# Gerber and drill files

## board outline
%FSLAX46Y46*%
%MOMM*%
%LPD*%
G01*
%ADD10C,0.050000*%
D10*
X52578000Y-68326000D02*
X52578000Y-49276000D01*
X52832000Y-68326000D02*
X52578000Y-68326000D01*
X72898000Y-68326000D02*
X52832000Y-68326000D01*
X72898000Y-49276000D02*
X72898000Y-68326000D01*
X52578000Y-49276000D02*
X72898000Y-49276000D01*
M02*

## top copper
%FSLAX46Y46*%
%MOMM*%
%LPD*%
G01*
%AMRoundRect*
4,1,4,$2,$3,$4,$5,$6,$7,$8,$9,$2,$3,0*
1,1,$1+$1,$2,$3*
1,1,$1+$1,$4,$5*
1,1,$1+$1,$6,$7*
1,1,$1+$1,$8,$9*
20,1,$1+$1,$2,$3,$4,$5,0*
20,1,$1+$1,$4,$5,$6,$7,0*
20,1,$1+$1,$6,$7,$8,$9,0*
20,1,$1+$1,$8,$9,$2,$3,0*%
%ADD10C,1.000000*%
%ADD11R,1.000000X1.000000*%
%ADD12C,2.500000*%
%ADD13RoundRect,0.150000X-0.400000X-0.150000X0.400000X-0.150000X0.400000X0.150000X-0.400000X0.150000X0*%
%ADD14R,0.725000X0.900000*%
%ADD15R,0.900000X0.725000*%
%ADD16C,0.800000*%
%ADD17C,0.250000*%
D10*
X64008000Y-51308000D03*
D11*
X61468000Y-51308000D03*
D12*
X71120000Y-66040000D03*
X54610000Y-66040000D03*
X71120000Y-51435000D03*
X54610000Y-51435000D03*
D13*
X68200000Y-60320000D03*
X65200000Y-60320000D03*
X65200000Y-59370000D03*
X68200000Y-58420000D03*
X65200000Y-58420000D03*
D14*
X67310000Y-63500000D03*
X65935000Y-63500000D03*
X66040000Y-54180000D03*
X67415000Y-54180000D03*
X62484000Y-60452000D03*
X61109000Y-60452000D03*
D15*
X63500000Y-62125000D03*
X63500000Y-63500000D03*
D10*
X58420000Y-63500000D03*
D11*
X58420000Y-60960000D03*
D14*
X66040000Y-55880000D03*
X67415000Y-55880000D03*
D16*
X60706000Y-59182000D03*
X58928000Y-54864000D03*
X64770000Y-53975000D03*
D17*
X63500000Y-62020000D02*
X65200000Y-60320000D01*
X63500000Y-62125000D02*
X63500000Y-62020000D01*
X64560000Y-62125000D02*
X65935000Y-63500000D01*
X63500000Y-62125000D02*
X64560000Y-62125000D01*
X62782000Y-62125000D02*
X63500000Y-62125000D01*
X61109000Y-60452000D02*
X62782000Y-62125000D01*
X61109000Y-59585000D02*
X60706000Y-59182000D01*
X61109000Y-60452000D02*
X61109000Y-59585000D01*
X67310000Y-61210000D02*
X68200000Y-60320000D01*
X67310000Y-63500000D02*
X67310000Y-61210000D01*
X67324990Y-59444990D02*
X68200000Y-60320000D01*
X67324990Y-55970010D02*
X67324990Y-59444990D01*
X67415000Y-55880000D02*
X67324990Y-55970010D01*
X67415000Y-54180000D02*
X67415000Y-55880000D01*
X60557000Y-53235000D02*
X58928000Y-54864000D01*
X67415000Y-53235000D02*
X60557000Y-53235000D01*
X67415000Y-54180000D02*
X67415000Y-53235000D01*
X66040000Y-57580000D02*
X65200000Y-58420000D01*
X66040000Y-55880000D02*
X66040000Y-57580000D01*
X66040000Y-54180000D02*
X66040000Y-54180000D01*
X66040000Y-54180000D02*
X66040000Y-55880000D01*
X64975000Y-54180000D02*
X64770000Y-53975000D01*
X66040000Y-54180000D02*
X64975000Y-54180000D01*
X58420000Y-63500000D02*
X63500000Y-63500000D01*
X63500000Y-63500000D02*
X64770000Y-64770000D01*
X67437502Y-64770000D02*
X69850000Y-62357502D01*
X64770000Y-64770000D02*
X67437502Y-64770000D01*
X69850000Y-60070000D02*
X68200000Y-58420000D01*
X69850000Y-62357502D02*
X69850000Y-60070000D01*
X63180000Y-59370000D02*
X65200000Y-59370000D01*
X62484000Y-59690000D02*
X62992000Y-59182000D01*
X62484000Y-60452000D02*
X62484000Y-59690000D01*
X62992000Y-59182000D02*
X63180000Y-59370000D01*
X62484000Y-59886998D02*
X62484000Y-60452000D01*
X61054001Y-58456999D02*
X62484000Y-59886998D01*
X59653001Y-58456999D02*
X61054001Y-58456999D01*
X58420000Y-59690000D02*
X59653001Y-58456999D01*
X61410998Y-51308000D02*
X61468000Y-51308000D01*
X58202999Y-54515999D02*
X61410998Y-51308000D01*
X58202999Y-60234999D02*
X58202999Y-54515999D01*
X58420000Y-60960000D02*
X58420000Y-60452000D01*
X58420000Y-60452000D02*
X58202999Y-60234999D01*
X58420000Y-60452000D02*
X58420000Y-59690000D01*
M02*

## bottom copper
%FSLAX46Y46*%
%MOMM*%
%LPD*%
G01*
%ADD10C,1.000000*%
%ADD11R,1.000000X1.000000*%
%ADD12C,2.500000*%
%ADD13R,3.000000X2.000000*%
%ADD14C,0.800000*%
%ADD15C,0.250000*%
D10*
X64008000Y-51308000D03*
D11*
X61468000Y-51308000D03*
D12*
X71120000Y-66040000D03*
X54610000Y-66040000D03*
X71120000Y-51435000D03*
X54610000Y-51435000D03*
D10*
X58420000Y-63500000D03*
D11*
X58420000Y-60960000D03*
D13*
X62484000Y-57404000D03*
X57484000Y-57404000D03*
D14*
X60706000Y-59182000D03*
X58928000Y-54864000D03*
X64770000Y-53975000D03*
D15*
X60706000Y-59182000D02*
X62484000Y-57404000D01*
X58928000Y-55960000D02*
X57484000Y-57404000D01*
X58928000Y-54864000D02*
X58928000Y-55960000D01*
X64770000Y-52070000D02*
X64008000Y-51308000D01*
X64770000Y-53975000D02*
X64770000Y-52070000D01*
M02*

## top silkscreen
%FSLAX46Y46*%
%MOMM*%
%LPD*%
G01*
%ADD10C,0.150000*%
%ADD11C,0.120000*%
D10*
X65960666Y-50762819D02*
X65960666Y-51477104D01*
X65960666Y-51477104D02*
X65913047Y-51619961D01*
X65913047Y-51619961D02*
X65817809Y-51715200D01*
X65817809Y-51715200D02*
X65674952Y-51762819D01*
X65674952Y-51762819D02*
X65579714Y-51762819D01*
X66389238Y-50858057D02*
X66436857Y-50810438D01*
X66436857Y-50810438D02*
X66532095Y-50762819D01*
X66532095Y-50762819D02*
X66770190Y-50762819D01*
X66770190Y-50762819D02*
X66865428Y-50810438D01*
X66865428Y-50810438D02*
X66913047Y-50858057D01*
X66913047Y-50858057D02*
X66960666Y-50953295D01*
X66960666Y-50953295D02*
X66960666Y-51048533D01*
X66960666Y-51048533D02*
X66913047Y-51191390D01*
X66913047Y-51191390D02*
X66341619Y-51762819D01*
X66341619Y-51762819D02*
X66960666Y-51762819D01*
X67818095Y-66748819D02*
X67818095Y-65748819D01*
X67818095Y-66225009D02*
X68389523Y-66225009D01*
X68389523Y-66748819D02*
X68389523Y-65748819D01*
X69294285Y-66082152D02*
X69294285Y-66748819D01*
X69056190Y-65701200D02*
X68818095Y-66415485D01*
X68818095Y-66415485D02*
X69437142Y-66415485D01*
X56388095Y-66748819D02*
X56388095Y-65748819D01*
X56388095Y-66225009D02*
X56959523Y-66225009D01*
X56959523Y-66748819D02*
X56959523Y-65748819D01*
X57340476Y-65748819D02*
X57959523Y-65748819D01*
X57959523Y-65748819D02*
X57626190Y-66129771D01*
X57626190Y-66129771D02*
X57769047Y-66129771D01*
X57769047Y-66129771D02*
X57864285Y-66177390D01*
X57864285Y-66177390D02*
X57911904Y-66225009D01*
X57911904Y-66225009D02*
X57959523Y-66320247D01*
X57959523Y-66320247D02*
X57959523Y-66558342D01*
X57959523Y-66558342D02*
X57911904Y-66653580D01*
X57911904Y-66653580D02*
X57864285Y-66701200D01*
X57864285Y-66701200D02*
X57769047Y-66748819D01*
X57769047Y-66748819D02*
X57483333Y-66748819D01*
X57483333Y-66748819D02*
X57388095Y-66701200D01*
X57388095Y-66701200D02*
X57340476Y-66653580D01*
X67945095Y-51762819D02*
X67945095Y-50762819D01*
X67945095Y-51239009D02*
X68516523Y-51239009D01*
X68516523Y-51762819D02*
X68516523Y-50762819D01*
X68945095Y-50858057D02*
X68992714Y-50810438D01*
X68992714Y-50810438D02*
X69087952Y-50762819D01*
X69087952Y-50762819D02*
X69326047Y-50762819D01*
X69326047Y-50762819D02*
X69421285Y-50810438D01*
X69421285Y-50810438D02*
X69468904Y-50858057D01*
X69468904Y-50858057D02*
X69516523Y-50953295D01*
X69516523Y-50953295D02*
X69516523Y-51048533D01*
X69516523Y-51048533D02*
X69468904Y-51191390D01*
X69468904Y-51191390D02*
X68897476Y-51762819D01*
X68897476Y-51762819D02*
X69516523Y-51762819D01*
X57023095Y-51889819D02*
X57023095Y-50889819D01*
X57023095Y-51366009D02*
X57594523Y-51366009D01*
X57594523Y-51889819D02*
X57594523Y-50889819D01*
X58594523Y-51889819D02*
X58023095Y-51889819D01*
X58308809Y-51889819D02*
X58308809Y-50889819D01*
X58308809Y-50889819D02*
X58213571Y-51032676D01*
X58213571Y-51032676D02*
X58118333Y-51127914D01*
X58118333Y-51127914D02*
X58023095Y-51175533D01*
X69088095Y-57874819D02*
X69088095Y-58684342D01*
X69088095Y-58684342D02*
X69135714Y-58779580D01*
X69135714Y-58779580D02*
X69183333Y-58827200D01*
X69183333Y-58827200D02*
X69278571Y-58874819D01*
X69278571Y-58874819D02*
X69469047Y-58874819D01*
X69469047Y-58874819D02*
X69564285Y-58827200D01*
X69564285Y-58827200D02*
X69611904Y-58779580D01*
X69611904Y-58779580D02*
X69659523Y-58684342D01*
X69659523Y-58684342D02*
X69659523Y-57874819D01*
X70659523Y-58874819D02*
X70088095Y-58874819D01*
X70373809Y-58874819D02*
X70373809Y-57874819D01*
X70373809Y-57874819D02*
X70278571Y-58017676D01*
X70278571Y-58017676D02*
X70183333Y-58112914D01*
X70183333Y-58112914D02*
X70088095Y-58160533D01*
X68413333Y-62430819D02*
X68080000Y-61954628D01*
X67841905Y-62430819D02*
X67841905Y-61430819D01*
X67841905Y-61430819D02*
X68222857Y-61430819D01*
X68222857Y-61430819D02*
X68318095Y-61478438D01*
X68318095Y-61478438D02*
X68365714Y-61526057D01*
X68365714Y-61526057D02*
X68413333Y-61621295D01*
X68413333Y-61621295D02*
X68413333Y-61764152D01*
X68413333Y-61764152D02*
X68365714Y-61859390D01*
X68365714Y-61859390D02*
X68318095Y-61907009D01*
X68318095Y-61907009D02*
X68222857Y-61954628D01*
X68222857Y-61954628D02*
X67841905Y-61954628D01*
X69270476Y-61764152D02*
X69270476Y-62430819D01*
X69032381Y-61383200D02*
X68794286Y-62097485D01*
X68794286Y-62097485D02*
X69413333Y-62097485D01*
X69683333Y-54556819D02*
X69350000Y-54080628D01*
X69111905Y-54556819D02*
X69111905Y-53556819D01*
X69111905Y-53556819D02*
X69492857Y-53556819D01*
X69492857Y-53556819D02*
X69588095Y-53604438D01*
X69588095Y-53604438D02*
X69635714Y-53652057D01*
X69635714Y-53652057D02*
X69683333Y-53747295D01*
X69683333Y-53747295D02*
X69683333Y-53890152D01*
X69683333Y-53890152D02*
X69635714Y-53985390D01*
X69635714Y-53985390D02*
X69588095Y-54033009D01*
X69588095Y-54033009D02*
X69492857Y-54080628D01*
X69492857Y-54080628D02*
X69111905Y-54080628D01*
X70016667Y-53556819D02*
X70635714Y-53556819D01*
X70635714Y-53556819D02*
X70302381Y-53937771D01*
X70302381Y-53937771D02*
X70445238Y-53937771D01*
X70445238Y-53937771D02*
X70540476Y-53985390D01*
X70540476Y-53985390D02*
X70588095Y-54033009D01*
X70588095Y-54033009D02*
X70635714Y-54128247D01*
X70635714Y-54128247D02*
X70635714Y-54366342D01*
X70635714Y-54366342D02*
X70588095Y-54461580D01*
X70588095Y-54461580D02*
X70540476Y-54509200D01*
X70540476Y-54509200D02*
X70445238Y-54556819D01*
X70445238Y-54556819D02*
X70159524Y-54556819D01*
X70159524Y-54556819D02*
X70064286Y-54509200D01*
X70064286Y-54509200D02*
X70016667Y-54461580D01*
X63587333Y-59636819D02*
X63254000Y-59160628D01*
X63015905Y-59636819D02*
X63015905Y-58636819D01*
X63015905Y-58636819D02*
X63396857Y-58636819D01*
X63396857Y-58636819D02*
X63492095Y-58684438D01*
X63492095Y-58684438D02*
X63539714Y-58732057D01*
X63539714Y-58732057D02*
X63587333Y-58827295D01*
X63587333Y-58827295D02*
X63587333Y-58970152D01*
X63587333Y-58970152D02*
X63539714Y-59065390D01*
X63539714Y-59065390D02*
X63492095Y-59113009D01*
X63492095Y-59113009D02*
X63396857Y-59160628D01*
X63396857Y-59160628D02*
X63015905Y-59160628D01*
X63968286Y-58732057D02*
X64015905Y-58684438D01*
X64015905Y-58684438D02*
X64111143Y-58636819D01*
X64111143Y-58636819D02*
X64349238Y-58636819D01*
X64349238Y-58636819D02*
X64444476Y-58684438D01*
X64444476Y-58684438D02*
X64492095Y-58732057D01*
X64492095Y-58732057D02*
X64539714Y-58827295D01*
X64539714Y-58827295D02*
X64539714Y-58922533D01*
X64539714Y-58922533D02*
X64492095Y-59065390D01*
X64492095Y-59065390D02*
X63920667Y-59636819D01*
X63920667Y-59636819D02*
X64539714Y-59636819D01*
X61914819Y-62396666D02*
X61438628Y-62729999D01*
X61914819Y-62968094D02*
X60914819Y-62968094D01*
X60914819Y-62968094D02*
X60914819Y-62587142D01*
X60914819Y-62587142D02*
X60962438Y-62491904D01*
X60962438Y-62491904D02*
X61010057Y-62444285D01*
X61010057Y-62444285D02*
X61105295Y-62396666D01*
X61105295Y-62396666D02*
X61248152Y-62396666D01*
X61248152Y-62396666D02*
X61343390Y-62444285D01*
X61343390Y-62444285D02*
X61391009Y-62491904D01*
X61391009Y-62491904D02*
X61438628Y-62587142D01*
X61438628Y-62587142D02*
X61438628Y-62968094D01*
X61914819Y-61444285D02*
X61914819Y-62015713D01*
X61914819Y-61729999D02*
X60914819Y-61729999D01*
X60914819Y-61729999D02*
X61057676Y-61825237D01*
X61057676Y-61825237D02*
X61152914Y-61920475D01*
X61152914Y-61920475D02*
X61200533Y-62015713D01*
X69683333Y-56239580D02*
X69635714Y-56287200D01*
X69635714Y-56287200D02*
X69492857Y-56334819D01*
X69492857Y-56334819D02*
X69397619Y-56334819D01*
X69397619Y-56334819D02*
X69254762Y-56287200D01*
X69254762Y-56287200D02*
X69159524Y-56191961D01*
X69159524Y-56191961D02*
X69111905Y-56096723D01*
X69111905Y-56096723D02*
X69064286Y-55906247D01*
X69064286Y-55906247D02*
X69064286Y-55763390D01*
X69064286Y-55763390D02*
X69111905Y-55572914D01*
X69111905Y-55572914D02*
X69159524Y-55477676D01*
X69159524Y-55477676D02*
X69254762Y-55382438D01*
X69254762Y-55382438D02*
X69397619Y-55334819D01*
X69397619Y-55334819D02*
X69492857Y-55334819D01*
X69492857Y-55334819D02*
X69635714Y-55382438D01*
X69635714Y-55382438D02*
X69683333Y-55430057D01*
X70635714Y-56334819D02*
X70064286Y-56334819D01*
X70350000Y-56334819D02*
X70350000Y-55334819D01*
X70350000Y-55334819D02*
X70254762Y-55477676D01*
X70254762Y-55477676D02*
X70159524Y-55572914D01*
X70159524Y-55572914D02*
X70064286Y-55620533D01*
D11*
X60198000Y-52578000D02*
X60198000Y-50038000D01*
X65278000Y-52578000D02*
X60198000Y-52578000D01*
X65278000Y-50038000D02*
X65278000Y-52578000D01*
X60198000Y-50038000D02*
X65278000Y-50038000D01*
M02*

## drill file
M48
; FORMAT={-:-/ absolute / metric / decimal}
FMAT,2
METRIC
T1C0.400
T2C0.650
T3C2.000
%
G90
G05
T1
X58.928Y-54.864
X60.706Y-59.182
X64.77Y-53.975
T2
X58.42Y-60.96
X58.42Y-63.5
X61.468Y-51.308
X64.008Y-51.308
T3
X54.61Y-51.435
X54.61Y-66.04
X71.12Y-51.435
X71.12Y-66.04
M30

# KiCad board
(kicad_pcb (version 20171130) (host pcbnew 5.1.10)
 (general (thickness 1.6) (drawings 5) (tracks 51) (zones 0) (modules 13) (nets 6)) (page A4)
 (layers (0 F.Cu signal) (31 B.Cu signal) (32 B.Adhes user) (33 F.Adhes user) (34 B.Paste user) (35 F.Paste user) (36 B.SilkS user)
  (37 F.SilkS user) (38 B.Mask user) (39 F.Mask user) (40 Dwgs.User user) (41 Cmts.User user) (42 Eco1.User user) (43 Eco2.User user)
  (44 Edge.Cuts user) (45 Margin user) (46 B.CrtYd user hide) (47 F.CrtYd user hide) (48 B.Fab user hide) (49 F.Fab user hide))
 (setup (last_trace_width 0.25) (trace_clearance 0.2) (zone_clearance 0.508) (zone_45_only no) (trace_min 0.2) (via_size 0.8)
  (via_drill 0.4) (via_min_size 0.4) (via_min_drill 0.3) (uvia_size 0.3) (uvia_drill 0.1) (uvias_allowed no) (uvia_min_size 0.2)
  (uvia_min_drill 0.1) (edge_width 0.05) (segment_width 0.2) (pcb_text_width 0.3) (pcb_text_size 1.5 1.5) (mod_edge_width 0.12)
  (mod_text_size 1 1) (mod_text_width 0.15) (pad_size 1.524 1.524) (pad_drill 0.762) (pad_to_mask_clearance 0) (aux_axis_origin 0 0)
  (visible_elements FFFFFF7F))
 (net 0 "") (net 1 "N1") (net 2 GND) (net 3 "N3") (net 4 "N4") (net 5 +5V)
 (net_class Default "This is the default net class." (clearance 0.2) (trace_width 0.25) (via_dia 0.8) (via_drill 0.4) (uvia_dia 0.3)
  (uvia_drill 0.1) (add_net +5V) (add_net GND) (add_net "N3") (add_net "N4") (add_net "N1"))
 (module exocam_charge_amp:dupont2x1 (layer F.Cu) (at 64.008 48.768)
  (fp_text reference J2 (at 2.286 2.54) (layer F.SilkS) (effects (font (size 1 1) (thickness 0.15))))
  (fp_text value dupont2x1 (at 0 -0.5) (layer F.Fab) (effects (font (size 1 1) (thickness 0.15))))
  (fp_line (start -3.81 3.81) (end -3.81 1.27) (layer F.SilkS) (width 0.12))
  (fp_line (start 1.27 3.81) (end -3.81 3.81) (layer F.SilkS) (width 0.12))
  (fp_line (start 1.27 1.27) (end 1.27 3.81) (layer F.SilkS) (width 0.12))
  (fp_line (start -3.81 1.27) (end 1.27 1.27) (layer F.SilkS) (width 0.12))
  (pad 2 thru_hole circle (at 0 2.54) (size 1 1) (drill 0.65) (layers *.Cu *.Mask) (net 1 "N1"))
  (pad 1 thru_hole rect (at -2.54 2.54) (size 1 1) (drill 0.65) (layers *.Cu *.Mask) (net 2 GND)))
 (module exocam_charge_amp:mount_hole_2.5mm (layer F.Cu) (at 72.39 62.23)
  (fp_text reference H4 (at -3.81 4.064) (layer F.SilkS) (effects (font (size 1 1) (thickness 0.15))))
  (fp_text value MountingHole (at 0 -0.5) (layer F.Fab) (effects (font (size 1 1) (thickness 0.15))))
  (pad 1 thru_hole circle (at -1.27 3.81) (size 2.5 2.5) (drill 2) (layers *.Cu *.Mask)))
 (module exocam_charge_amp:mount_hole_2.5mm (layer F.Cu) (at 55.88 62.23)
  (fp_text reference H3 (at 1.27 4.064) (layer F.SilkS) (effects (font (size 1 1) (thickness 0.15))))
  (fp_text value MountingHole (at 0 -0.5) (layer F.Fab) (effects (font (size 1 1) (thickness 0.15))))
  (pad 1 thru_hole circle (at -1.27 3.81) (size 2.5 2.5) (drill 2) (layers *.Cu *.Mask)))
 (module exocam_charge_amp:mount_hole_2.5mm (layer F.Cu) (at 72.39 47.625)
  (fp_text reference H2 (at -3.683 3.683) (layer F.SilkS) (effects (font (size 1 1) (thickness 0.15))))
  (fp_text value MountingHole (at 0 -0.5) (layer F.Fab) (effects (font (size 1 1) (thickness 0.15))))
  (pad 1 thru_hole circle (at -1.27 3.81) (size 2.5 2.5) (drill 2) (layers *.Cu *.Mask)))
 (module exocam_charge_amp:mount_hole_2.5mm (layer F.Cu) (at 55.88 47.625)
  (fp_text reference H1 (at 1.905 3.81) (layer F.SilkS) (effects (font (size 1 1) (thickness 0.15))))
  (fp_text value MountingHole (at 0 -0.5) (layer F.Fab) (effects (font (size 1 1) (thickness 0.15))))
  (pad 1 thru_hole circle (at -1.27 3.81) (size 2.5 2.5) (drill 2) (layers *.Cu *.Mask)))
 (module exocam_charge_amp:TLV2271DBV (layer F.Cu) (at 66.47 55.88)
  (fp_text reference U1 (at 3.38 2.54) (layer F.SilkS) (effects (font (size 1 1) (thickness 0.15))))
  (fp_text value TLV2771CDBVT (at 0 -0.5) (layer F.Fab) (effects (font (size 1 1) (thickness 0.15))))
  (pad 4 smd roundrect (at 1.73 4.44) (size 1.1 0.6) (layers F.Cu F.Paste F.Mask) (roundrect_rratio 0.25) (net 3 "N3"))
  (pad 3 smd roundrect (at -1.27 4.44) (size 1.1 0.6) (layers F.Cu F.Paste F.Mask) (roundrect_rratio 0.25) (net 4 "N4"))
  (pad 2 smd roundrect (at -1.27 3.49) (size 1.1 0.6) (layers F.Cu F.Paste F.Mask) (roundrect_rratio 0.25) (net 2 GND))
  (pad 5 smd roundrect (at 1.73 2.54) (size 1.1 0.6) (layers F.Cu F.Paste F.Mask) (roundrect_rratio 0.25) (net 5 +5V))
  (pad 1 smd roundrect (at -1.27 2.54) (size 1.1 0.6) (layers F.Cu F.Paste F.Mask) (roundrect_rratio 0.25) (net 1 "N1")))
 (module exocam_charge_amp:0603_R (layer F.Cu) (at 67.205 60.96)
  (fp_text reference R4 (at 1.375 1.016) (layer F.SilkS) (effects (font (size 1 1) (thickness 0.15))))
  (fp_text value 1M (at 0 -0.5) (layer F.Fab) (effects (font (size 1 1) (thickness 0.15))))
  (pad 2 smd rect (at 0.105 2.54) (size 0.725 0.9) (layers F.Cu F.Paste F.Mask) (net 3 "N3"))
  (pad 1 smd rect (at -1.27 2.54) (size 0.725 0.9) (layers F.Cu F.Paste F.Mask) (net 4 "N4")))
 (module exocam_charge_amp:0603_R (layer F.Cu) (at 66.145 56.72 180)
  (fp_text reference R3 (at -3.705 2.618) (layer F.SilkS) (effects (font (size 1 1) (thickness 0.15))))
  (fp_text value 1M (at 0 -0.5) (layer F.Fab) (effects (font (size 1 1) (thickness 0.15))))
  (pad 2 smd rect (at 0.105 2.54 180) (size 0.725 0.9) (layers F.Cu F.Paste F.Mask) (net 1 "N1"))
  (pad 1 smd rect (at -1.27 2.54 180) (size 0.725 0.9) (layers F.Cu F.Paste F.Mask) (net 3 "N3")))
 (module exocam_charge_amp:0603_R (layer F.Cu) (at 62.379 57.912)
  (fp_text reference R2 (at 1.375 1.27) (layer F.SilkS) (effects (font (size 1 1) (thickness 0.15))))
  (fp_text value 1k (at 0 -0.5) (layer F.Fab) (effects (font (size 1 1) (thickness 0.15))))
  (pad 2 smd rect (at 0.105 2.54) (size 0.725 0.9) (layers F.Cu F.Paste F.Mask) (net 2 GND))
  (pad 1 smd rect (at -1.27 2.54) (size 0.725 0.9) (layers F.Cu F.Paste F.Mask) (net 4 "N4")))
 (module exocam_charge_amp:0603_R (layer F.Cu) (at 60.96 62.23 90)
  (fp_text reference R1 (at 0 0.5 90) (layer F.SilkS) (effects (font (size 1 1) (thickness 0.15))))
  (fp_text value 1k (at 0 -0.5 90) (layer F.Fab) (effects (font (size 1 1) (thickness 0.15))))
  (pad 2 smd rect (at 0.105 2.54 90) (size 0.725 0.9) (layers F.Cu F.Paste F.Mask) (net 4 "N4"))
  (pad 1 smd rect (at -1.27 2.54 90) (size 0.725 0.9) (layers F.Cu F.Paste F.Mask) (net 5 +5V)))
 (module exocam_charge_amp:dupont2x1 (layer B.Cu) (at 55.88 63.5 270)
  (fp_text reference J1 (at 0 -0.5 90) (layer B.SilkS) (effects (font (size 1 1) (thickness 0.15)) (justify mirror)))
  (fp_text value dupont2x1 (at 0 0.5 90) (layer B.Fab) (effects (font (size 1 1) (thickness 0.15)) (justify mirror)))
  (pad 2 thru_hole circle (at 0 -2.54 270) (size 1 1) (drill 0.65) (layers *.Cu *.Mask) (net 5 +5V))
  (pad 1 thru_hole rect (at -2.54 -2.54 270) (size 1 1) (drill 0.65) (layers *.Cu *.Mask) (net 2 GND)))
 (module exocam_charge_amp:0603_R (layer F.Cu) (at 66.145 58.42 180)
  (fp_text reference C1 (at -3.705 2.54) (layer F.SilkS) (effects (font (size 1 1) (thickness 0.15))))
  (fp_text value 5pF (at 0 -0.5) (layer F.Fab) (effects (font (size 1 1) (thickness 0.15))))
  (pad 2 smd rect (at 0.105 2.54 180) (size 0.725 0.9) (layers F.Cu F.Paste F.Mask) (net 1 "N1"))
  (pad 1 smd rect (at -1.27 2.54 180) (size 0.725 0.9) (layers F.Cu F.Paste F.Mask) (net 3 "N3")))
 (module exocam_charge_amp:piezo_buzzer (layer B.Cu) (at 60.024 59.944)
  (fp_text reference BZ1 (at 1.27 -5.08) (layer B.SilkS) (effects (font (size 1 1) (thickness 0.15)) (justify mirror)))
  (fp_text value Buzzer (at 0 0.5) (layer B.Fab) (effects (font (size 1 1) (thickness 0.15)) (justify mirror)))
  (pad 2 smd rect (at 2.46 -2.54) (size 3 2) (layers B.Cu B.Paste B.Mask) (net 4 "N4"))
  (pad 1 smd rect (at -2.54 -2.54) (size 3 2) (layers B.Cu B.Paste B.Mask) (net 3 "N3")))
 (gr_line (start 52.578 68.326) (end 52.578 49.276) (layer Edge.Cuts) (width 0.05))
 (gr_line (start 52.832 68.326) (end 52.578 68.326) (layer Edge.Cuts) (width 0.05))
 (gr_line (start 72.898 68.326) (end 52.832 68.326) (layer Edge.Cuts) (width 0.05))
 (gr_line (start 72.898 49.276) (end 72.898 68.326) (layer Edge.Cuts) (width 0.05))
 (gr_line (start 52.578 49.276) (end 72.898 49.276) (layer Edge.Cuts) (width 0.05))
 (segment (start 63.5 62.02) (end 65.2 60.32) (width 0.25) (layer F.Cu) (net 4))
 (segment (start 63.5 62.125) (end 63.5 62.02) (width 0.25) (layer F.Cu) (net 4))
 (segment (start 64.56 62.125) (end 65.935 63.5) (width 0.25) (layer F.Cu) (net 4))
 (segment (start 63.5 62.125) (end 64.56 62.125) (width 0.25) (layer F.Cu) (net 4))
 (via (at 60.706 59.182) (size 0.8) (drill 0.4) (layers F.Cu B.Cu) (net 4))
 (segment (start 62.782 62.125) (end 63.5 62.125) (width 0.25) (layer F.Cu) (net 4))
 (segment (start 61.109 60.452) (end 62.782 62.125) (width 0.25) (layer F.Cu) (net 4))
 (segment (start 60.706 59.182) (end 62.484 57.404) (width 0.25) (layer B.Cu) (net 4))
 (segment (start 61.109 59.585) (end 60.706 59.182) (width 0.25) (layer F.Cu) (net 4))
 (segment (start 61.109 60.452) (end 61.109 59.585) (width 0.25) (layer F.Cu) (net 4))
 (via (at 58.928 54.864) (size 0.8) (drill 0.4) (layers F.Cu B.Cu) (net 3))
 (segment (start 67.31 61.21) (end 68.2 60.32) (width 0.25) (layer F.Cu) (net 3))
 (segment (start 67.31 63.5) (end 67.31 61.21) (width 0.25) (layer F.Cu) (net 3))
 (segment (start 67.32499 59.44499) (end 68.2 60.32) (width 0.25) (layer F.Cu) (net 3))
 (segment (start 67.32499 55.97001) (end 67.32499 59.44499) (width 0.25) (layer F.Cu) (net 3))
 (segment (start 67.415 55.88) (end 67.32499 55.97001) (width 0.25) (layer F.Cu) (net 3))
 (segment (start 67.415 54.18) (end 67.415 55.88) (width 0.25) (layer F.Cu) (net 3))
 (segment (start 60.557 53.235) (end 58.928 54.864) (width 0.25) (layer F.Cu) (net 3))
 (segment (start 67.415 53.235) (end 60.557 53.235) (width 0.25) (layer F.Cu) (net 3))
 (segment (start 67.415 54.18) (end 67.415 53.235) (width 0.25) (layer F.Cu) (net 3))
 (segment (start 58.928 55.96) (end 57.484 57.404) (width 0.25) (layer B.Cu) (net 3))
 (segment (start 58.928 54.864) (end 58.928 55.96) (width 0.25) (layer B.Cu) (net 3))
 (segment (start 66.04 57.58) (end 65.2 58.42) (width 0.25) (layer F.Cu) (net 1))
 (segment (start 66.04 55.88) (end 66.04 57.58) (width 0.25) (layer F.Cu) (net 1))
 (segment (start 66.04 54.18) (end 66.04 54.18) (width 0.25) (layer F.Cu) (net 1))
 (segment (start 66.04 54.18) (end 66.04 55.88) (width 0.25) (layer F.Cu) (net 1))
 (via (at 64.77 53.975) (size 0.8) (drill 0.4) (layers F.Cu B.Cu) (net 1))
 (segment (start 64.975 54.18) (end 64.77 53.975) (width 0.25) (layer F.Cu) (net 1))
 (segment (start 66.04 54.18) (end 64.975 54.18) (width 0.25) (layer F.Cu) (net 1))
 (segment (start 64.77 52.07) (end 64.008 51.308) (width 0.25) (layer B.Cu) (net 1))
 (segment (start 64.77 53.975) (end 64.77 52.07) (width 0.25) (layer B.Cu) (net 1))
 (segment (start 58.42 63.5) (end 63.5 63.5) (width 0.25) (layer F.Cu) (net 5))
 (segment (start 63.5 63.5) (end 64.77 64.77) (width 0.25) (layer F.Cu) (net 5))
 (segment (start 67.437502 64.77) (end 69.85 62.357502) (width 0.25) (layer F.Cu) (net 5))
 (segment (start 64.77 64.77) (end 67.437502 64.77) (width 0.25) (layer F.Cu) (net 5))
 (segment (start 69.85 60.07) (end 68.2 58.42) (width 0.25) (layer F.Cu) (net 5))
 (segment (start 69.85 62.357502) (end 69.85 60.07) (width 0.25) (layer F.Cu) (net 5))
 (segment (start 63.18 59.37) (end 65.2 59.37) (width 0.25) (layer F.Cu) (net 2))
 (segment (start 62.484 59.69) (end 62.992 59.182) (width 0.25) (layer F.Cu) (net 2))
 (segment (start 62.484 60.452) (end 62.484 59.69) (width 0.25) (layer F.Cu) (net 2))
 (segment (start 62.992 59.182) (end 63.18 59.37) (width 0.25) (layer F.Cu) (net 2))
 (segment (start 62.484 59.886998) (end 62.484 60.452) (width 0.25) (layer F.Cu) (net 2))
 (segment (start 61.054001 58.456999) (end 62.484 59.886998) (width 0.25) (layer F.Cu) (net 2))
 (segment (start 59.653001 58.456999) (end 61.054001 58.456999) (width 0.25) (layer F.Cu) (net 2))
 (segment (start 58.42 59.69) (end 59.653001 58.456999) (width 0.25) (layer F.Cu) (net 2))
 (segment (start 61.410998 51.308) (end 61.468 51.308) (width 0.25) (layer F.Cu) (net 2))
 (segment (start 58.202999 54.515999) (end 61.410998 51.308) (width 0.25) (layer F.Cu) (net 2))
 (segment (start 58.202999 60.234999) (end 58.202999 54.515999) (width 0.25) (layer F.Cu) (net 2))
 (segment (start 58.42 60.96) (end 58.42 60.452) (width 0.25) (layer F.Cu) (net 2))
 (segment (start 58.42 60.452) (end 58.202999 60.234999) (width 0.25) (layer F.Cu) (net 2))
 (segment (start 58.42 60.452) (end 58.42 59.69) (width 0.25) (layer F.Cu) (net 2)))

